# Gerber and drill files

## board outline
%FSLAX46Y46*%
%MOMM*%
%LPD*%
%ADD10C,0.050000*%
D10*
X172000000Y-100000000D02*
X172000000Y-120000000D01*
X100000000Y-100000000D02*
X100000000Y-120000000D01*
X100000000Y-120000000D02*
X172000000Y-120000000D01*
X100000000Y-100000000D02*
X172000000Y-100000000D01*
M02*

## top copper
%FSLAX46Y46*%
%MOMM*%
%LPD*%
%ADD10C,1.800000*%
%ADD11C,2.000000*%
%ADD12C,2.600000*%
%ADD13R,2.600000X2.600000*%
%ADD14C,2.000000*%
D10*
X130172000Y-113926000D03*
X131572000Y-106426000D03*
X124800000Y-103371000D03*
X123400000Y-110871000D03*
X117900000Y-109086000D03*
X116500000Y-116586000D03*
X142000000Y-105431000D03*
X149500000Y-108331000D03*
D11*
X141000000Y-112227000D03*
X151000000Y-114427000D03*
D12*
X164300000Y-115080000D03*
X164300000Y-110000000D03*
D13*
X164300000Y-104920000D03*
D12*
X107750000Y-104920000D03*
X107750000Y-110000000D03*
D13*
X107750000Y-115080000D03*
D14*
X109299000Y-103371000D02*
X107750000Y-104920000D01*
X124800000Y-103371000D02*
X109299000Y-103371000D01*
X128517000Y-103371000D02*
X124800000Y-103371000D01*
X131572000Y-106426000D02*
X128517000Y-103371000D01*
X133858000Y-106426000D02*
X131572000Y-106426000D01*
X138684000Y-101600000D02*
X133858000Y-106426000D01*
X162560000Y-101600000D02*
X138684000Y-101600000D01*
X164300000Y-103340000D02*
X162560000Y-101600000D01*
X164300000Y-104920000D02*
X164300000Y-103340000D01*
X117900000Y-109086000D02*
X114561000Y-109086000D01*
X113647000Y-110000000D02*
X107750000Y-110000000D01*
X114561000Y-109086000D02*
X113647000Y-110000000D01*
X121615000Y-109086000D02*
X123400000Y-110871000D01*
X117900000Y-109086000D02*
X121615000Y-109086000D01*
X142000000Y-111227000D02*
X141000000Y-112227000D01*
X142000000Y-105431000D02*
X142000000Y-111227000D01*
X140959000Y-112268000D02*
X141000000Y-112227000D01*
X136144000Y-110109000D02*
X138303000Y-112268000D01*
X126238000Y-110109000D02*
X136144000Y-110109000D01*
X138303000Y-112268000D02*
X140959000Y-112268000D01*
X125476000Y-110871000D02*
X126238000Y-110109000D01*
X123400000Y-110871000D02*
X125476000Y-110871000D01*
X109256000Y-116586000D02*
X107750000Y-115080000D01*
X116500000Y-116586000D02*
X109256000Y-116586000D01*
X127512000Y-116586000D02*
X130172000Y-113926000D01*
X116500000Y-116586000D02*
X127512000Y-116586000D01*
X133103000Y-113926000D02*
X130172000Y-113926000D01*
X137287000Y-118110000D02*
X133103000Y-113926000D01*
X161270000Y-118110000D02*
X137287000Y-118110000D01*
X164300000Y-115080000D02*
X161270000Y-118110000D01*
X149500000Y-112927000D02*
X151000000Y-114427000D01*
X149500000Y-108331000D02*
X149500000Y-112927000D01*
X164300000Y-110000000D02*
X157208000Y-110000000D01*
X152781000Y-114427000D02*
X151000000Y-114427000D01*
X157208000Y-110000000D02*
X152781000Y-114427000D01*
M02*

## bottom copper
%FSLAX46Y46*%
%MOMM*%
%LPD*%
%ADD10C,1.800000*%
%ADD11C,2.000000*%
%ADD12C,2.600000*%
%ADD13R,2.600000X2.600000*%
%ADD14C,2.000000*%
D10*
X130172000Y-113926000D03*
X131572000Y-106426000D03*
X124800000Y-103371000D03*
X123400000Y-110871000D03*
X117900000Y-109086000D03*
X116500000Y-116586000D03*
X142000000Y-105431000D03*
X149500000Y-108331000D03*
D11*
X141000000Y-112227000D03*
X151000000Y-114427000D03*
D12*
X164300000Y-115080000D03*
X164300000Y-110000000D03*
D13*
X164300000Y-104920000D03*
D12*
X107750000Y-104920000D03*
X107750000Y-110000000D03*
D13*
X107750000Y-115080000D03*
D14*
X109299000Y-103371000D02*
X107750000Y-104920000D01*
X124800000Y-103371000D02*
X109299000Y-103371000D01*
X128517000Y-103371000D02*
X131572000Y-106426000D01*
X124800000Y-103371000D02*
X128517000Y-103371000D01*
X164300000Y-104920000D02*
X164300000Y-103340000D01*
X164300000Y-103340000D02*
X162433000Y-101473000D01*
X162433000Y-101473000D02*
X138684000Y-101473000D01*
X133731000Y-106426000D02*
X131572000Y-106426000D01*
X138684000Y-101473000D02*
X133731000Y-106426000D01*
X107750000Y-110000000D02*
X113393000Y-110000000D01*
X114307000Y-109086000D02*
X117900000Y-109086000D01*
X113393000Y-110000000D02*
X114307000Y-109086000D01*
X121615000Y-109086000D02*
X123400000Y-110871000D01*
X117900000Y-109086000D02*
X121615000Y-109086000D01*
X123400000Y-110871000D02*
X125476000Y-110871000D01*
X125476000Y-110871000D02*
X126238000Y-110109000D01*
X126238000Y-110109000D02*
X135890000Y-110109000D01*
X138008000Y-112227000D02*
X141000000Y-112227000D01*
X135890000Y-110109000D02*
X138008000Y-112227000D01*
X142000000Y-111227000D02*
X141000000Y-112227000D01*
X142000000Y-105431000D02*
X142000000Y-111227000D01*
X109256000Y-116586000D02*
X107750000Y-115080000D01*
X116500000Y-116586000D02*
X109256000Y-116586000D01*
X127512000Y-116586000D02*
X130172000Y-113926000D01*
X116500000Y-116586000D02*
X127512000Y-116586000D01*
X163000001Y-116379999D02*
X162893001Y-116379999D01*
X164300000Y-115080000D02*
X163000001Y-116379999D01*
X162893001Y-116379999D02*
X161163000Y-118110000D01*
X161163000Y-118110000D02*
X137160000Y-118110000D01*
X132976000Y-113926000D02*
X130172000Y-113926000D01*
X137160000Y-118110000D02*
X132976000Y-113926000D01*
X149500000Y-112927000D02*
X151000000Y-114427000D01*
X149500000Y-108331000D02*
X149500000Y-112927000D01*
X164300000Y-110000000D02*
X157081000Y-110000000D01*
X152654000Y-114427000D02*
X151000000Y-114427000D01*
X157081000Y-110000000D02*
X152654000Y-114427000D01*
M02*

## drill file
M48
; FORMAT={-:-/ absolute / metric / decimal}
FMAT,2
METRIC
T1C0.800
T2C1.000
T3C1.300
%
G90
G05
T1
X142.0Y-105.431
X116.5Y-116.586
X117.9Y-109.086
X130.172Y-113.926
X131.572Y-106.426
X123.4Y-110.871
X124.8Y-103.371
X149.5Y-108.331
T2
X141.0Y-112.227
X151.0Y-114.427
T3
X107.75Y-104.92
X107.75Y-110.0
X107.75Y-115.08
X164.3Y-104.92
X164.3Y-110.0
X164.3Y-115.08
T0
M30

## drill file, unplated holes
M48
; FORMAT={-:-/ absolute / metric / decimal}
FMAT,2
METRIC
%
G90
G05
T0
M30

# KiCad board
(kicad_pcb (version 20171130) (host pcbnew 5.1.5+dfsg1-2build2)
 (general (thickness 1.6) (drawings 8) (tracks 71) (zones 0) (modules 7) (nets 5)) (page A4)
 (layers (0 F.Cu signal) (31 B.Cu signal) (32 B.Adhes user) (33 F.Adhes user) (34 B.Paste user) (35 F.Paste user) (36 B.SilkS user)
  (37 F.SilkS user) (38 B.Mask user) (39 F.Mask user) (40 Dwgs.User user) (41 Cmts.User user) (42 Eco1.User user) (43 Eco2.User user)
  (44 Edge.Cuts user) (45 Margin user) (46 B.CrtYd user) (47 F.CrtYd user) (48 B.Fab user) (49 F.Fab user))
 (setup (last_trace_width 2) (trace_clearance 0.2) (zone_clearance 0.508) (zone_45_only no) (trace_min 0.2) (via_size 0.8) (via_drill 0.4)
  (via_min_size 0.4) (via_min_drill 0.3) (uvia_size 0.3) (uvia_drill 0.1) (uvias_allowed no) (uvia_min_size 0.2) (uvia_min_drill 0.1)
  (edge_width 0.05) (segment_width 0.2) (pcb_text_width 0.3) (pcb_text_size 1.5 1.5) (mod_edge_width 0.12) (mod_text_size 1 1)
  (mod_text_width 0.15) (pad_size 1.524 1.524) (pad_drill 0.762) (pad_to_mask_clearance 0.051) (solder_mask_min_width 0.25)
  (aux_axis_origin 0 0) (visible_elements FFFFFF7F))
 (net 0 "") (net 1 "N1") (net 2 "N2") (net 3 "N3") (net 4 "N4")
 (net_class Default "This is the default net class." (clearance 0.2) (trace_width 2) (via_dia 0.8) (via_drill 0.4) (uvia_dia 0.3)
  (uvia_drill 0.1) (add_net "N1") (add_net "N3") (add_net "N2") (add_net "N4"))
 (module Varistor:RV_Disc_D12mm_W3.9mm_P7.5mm (layer F.Cu) (at 131.572 106.426 270)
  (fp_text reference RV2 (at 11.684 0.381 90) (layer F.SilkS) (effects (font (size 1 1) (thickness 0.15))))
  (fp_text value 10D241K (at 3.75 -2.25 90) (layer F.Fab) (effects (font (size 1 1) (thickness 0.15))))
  (pad 2 thru_hole circle (at 7.5 1.4 270) (size 1.8 1.8) (drill 0.8) (layers *.Cu *.Mask) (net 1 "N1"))
  (pad 1 thru_hole circle (at 0 0 270) (size 1.8 1.8) (drill 0.8) (layers *.Cu *.Mask) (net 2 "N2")))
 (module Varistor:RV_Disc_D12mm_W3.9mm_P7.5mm (layer F.Cu) (at 123.4 110.871 90)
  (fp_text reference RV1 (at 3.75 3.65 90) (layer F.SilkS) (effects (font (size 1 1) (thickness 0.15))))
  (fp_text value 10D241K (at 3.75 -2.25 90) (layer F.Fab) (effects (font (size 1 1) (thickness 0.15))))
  (pad 2 thru_hole circle (at 7.5 1.4 90) (size 1.8 1.8) (drill 0.8) (layers *.Cu *.Mask) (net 2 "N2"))
  (pad 1 thru_hole circle (at 0 0 90) (size 1.8 1.8) (drill 0.8) (layers *.Cu *.Mask) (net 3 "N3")))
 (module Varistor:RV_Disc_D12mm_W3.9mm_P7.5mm (layer F.Cu) (at 116.5 116.586 90)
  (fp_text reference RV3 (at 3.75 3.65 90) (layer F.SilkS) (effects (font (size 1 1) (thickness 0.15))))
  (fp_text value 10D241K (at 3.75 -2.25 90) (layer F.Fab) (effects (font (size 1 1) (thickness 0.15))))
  (pad 2 thru_hole circle (at 7.5 1.4 90) (size 1.8 1.8) (drill 0.8) (layers *.Cu *.Mask) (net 3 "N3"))
  (pad 1 thru_hole circle (at 0 0 90) (size 1.8 1.8) (drill 0.8) (layers *.Cu *.Mask) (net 1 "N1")))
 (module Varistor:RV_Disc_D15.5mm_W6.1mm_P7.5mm (layer F.Cu) (at 149.5 108.331 180)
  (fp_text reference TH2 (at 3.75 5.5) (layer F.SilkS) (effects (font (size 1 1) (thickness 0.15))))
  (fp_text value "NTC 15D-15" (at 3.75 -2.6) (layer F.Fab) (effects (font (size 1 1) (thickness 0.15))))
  (pad 2 thru_hole circle (at 7.5 2.9 180) (size 1.8 1.8) (drill 0.8) (layers *.Cu *.Mask) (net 3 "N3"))
  (pad 1 thru_hole circle (at 0 0 180) (size 1.8 1.8) (drill 0.8) (layers *.Cu *.Mask) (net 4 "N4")))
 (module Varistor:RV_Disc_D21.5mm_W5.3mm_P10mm (layer F.Cu) (at 151 114.427 180)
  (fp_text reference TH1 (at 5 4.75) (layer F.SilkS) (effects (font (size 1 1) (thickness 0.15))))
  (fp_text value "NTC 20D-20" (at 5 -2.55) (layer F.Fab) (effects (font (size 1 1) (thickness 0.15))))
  (pad 2 thru_hole circle (at 10 2.2 180) (size 2 2) (drill 1) (layers *.Cu *.Mask) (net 3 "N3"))
  (pad 1 thru_hole circle (at 0 0 180) (size 2 2) (drill 1) (layers *.Cu *.Mask) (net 4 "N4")))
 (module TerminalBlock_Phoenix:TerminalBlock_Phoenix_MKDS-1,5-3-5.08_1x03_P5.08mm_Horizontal (layer F.Cu) (at 164.3 104.92 270)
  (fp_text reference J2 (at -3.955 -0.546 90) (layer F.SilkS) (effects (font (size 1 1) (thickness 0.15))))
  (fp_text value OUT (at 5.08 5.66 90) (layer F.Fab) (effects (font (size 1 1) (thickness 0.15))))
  (pad 3 thru_hole circle (at 10.16 0 270) (size 2.6 2.6) (drill 1.3) (layers *.Cu *.Mask) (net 1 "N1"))
  (pad 2 thru_hole circle (at 5.08 0 270) (size 2.6 2.6) (drill 1.3) (layers *.Cu *.Mask) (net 4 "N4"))
  (pad 1 thru_hole rect (at 0 0 270) (size 2.6 2.6) (drill 1.3) (layers *.Cu *.Mask) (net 2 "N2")))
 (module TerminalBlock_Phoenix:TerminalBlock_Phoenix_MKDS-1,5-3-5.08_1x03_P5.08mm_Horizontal (layer F.Cu) (at 107.75 115.08 90)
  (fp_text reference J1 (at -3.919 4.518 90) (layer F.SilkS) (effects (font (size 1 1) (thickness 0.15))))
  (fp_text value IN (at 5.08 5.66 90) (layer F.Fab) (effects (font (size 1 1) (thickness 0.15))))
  (pad 3 thru_hole circle (at 10.16 0 90) (size 2.6 2.6) (drill 1.3) (layers *.Cu *.Mask) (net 2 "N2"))
  (pad 2 thru_hole circle (at 5.08 0 90) (size 2.6 2.6) (drill 1.3) (layers *.Cu *.Mask) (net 3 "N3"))
  (pad 1 thru_hole rect (at 0 0 90) (size 2.6 2.6) (drill 1.3) (layers *.Cu *.Mask) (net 1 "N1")))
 (gr_line (start 172 100) (end 172 120) (layer Edge.Cuts) (width 0.05))
 (gr_line (start 100 100) (end 100 120) (layer Edge.Cuts) (width 0.05))
 (gr_line (start 100 120) (end 172 120) (layer Edge.Cuts) (width 0.05))
 (gr_line (start 100 100) (end 172 100) (layer Edge.Cuts) (width 0.05))
 (segment (start 109.299 103.371) (end 107.75 104.92) (width 2) (layer F.Cu) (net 2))
 (segment (start 124.8 103.371) (end 109.299 103.371) (width 2) (layer F.Cu) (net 2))
 (segment (start 128.517 103.371) (end 124.8 103.371) (width 2) (layer F.Cu) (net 2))
 (segment (start 131.572 106.426) (end 128.517 103.371) (width 2) (layer F.Cu) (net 2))
 (segment (start 133.858 106.426) (end 131.572 106.426) (width 2) (layer F.Cu) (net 2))
 (segment (start 138.684 101.6) (end 133.858 106.426) (width 2) (layer F.Cu) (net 2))
 (segment (start 162.56 101.6) (end 138.684 101.6) (width 2) (layer F.Cu) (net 2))
 (segment (start 164.3 103.34) (end 162.56 101.6) (width 2) (layer F.Cu) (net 2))
 (segment (start 164.3 104.92) (end 164.3 103.34) (width 2) (layer F.Cu) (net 2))
 (segment (start 109.299 103.371) (end 107.75 104.92) (width 2) (layer B.Cu) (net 2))
 (segment (start 124.8 103.371) (end 109.299 103.371) (width 2) (layer B.Cu) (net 2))
 (segment (start 128.517 103.371) (end 131.572 106.426) (width 2) (layer B.Cu) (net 2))
 (segment (start 124.8 103.371) (end 128.517 103.371) (width 2) (layer B.Cu) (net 2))
 (segment (start 164.3 104.92) (end 164.3 103.34) (width 2) (layer B.Cu) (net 2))
 (segment (start 164.3 103.34) (end 162.433 101.473) (width 2) (layer B.Cu) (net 2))
 (segment (start 162.433 101.473) (end 138.684 101.473) (width 2) (layer B.Cu) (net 2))
 (segment (start 133.731 106.426) (end 131.572 106.426) (width 2) (layer B.Cu) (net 2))
 (segment (start 138.684 101.473) (end 133.731 106.426) (width 2) (layer B.Cu) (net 2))
 (segment (start 117.9 109.086) (end 114.561 109.086) (width 2) (layer F.Cu) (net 3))
 (segment (start 113.647 110) (end 107.75 110) (width 2) (layer F.Cu) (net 3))
 (segment (start 114.561 109.086) (end 113.647 110) (width 2) (layer F.Cu) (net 3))
 (segment (start 121.615 109.086) (end 123.4 110.871) (width 2) (layer F.Cu) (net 3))
 (segment (start 117.9 109.086) (end 121.615 109.086) (width 2) (layer F.Cu) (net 3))
 (segment (start 142 111.227) (end 141 112.227) (width 2) (layer F.Cu) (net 3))
 (segment (start 142 105.431) (end 142 111.227) (width 2) (layer F.Cu) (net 3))
 (segment (start 140.959 112.268) (end 141 112.227) (width 2) (layer F.Cu) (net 3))
 (segment (start 136.144 110.109) (end 138.303 112.268) (width 2) (layer F.Cu) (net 3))
 (segment (start 126.238 110.109) (end 136.144 110.109) (width 2) (layer F.Cu) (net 3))
 (segment (start 138.303 112.268) (end 140.959 112.268) (width 2) (layer F.Cu) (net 3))
 (segment (start 125.476 110.871) (end 126.238 110.109) (width 2) (layer F.Cu) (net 3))
 (segment (start 123.4 110.871) (end 125.476 110.871) (width 2) (layer F.Cu) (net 3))
 (segment (start 107.75 110) (end 113.393 110) (width 2) (layer B.Cu) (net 3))
 (segment (start 114.307 109.086) (end 117.9 109.086) (width 2) (layer B.Cu) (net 3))
 (segment (start 113.393 110) (end 114.307 109.086) (width 2) (layer B.Cu) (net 3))
 (segment (start 121.615 109.086) (end 123.4 110.871) (width 2) (layer B.Cu) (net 3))
 (segment (start 117.9 109.086) (end 121.615 109.086) (width 2) (layer B.Cu) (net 3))
 (segment (start 123.4 110.871) (end 125.476 110.871) (width 2) (layer B.Cu) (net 3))
 (segment (start 125.476 110.871) (end 126.238 110.109) (width 2) (layer B.Cu) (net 3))
 (segment (start 126.238 110.109) (end 135.89 110.109) (width 2) (layer B.Cu) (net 3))
 (segment (start 138.008 112.227) (end 141 112.227) (width 2) (layer B.Cu) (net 3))
 (segment (start 135.89 110.109) (end 138.008 112.227) (width 2) (layer B.Cu) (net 3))
 (segment (start 142 111.227) (end 141 112.227) (width 2) (layer B.Cu) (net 3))
 (segment (start 142 105.431) (end 142 111.227) (width 2) (layer B.Cu) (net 3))
 (segment (start 109.256 116.586) (end 107.75 115.08) (width 2) (layer F.Cu) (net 1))
 (segment (start 116.5 116.586) (end 109.256 116.586) (width 2) (layer F.Cu) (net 1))
 (segment (start 127.512 116.586) (end 130.172 113.926) (width 2) (layer F.Cu) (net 1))
 (segment (start 116.5 116.586) (end 127.512 116.586) (width 2) (layer F.Cu) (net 1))
 (segment (start 133.103 113.926) (end 130.172 113.926) (width 2) (layer F.Cu) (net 1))
 (segment (start 137.287 118.11) (end 133.103 113.926) (width 2) (layer F.Cu) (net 1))
 (segment (start 161.27 118.11) (end 137.287 118.11) (width 2) (layer F.Cu) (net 1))
 (segment (start 164.3 115.08) (end 161.27 118.11) (width 2) (layer F.Cu) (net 1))
 (segment (start 109.256 116.586) (end 107.75 115.08) (width 2) (layer B.Cu) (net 1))
 (segment (start 116.5 116.586) (end 109.256 116.586) (width 2) (layer B.Cu) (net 1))
 (segment (start 127.512 116.586) (end 130.172 113.926) (width 2) (layer B.Cu) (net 1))
 (segment (start 116.5 116.586) (end 127.512 116.586) (width 2) (layer B.Cu) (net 1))
 (segment (start 163.000001 116.379999) (end 162.893001 116.379999) (width 2) (layer B.Cu) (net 1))
 (segment (start 164.3 115.08) (end 163.000001 116.379999) (width 2) (layer B.Cu) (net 1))
 (segment (start 162.893001 116.379999) (end 161.163 118.11) (width 2) (layer B.Cu) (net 1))
 (segment (start 161.163 118.11) (end 137.16 118.11) (width 2) (layer B.Cu) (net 1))
 (segment (start 132.976 113.926) (end 130.172 113.926) (width 2) (layer B.Cu) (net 1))
 (segment (start 137.16 118.11) (end 132.976 113.926) (width 2) (layer B.Cu) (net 1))
 (segment (start 149.5 112.927) (end 151 114.427) (width 2) (layer F.Cu) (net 4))
 (segment (start 149.5 108.331) (end 149.5 112.927) (width 2) (layer F.Cu) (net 4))
 (segment (start 164.3 110) (end 157.208 110) (width 2) (layer F.Cu) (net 4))
 (segment (start 152.781 114.427) (end 151 114.427) (width 2) (layer F.Cu) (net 4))
 (segment (start 157.208 110) (end 152.781 114.427) (width 2) (layer F.Cu) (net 4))
 (segment (start 149.5 112.927) (end 151 114.427) (width 2) (layer B.Cu) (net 4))
 (segment (start 149.5 108.331) (end 149.5 112.927) (width 2) (layer B.Cu) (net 4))
 (segment (start 164.3 110) (end 157.081 110) (width 2) (layer B.Cu) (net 4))
 (segment (start 152.654 114.427) (end 151 114.427) (width 2) (layer B.Cu) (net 4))
 (segment (start 157.081 110) (end 152.654 114.427) (width 2) (layer B.Cu) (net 4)))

